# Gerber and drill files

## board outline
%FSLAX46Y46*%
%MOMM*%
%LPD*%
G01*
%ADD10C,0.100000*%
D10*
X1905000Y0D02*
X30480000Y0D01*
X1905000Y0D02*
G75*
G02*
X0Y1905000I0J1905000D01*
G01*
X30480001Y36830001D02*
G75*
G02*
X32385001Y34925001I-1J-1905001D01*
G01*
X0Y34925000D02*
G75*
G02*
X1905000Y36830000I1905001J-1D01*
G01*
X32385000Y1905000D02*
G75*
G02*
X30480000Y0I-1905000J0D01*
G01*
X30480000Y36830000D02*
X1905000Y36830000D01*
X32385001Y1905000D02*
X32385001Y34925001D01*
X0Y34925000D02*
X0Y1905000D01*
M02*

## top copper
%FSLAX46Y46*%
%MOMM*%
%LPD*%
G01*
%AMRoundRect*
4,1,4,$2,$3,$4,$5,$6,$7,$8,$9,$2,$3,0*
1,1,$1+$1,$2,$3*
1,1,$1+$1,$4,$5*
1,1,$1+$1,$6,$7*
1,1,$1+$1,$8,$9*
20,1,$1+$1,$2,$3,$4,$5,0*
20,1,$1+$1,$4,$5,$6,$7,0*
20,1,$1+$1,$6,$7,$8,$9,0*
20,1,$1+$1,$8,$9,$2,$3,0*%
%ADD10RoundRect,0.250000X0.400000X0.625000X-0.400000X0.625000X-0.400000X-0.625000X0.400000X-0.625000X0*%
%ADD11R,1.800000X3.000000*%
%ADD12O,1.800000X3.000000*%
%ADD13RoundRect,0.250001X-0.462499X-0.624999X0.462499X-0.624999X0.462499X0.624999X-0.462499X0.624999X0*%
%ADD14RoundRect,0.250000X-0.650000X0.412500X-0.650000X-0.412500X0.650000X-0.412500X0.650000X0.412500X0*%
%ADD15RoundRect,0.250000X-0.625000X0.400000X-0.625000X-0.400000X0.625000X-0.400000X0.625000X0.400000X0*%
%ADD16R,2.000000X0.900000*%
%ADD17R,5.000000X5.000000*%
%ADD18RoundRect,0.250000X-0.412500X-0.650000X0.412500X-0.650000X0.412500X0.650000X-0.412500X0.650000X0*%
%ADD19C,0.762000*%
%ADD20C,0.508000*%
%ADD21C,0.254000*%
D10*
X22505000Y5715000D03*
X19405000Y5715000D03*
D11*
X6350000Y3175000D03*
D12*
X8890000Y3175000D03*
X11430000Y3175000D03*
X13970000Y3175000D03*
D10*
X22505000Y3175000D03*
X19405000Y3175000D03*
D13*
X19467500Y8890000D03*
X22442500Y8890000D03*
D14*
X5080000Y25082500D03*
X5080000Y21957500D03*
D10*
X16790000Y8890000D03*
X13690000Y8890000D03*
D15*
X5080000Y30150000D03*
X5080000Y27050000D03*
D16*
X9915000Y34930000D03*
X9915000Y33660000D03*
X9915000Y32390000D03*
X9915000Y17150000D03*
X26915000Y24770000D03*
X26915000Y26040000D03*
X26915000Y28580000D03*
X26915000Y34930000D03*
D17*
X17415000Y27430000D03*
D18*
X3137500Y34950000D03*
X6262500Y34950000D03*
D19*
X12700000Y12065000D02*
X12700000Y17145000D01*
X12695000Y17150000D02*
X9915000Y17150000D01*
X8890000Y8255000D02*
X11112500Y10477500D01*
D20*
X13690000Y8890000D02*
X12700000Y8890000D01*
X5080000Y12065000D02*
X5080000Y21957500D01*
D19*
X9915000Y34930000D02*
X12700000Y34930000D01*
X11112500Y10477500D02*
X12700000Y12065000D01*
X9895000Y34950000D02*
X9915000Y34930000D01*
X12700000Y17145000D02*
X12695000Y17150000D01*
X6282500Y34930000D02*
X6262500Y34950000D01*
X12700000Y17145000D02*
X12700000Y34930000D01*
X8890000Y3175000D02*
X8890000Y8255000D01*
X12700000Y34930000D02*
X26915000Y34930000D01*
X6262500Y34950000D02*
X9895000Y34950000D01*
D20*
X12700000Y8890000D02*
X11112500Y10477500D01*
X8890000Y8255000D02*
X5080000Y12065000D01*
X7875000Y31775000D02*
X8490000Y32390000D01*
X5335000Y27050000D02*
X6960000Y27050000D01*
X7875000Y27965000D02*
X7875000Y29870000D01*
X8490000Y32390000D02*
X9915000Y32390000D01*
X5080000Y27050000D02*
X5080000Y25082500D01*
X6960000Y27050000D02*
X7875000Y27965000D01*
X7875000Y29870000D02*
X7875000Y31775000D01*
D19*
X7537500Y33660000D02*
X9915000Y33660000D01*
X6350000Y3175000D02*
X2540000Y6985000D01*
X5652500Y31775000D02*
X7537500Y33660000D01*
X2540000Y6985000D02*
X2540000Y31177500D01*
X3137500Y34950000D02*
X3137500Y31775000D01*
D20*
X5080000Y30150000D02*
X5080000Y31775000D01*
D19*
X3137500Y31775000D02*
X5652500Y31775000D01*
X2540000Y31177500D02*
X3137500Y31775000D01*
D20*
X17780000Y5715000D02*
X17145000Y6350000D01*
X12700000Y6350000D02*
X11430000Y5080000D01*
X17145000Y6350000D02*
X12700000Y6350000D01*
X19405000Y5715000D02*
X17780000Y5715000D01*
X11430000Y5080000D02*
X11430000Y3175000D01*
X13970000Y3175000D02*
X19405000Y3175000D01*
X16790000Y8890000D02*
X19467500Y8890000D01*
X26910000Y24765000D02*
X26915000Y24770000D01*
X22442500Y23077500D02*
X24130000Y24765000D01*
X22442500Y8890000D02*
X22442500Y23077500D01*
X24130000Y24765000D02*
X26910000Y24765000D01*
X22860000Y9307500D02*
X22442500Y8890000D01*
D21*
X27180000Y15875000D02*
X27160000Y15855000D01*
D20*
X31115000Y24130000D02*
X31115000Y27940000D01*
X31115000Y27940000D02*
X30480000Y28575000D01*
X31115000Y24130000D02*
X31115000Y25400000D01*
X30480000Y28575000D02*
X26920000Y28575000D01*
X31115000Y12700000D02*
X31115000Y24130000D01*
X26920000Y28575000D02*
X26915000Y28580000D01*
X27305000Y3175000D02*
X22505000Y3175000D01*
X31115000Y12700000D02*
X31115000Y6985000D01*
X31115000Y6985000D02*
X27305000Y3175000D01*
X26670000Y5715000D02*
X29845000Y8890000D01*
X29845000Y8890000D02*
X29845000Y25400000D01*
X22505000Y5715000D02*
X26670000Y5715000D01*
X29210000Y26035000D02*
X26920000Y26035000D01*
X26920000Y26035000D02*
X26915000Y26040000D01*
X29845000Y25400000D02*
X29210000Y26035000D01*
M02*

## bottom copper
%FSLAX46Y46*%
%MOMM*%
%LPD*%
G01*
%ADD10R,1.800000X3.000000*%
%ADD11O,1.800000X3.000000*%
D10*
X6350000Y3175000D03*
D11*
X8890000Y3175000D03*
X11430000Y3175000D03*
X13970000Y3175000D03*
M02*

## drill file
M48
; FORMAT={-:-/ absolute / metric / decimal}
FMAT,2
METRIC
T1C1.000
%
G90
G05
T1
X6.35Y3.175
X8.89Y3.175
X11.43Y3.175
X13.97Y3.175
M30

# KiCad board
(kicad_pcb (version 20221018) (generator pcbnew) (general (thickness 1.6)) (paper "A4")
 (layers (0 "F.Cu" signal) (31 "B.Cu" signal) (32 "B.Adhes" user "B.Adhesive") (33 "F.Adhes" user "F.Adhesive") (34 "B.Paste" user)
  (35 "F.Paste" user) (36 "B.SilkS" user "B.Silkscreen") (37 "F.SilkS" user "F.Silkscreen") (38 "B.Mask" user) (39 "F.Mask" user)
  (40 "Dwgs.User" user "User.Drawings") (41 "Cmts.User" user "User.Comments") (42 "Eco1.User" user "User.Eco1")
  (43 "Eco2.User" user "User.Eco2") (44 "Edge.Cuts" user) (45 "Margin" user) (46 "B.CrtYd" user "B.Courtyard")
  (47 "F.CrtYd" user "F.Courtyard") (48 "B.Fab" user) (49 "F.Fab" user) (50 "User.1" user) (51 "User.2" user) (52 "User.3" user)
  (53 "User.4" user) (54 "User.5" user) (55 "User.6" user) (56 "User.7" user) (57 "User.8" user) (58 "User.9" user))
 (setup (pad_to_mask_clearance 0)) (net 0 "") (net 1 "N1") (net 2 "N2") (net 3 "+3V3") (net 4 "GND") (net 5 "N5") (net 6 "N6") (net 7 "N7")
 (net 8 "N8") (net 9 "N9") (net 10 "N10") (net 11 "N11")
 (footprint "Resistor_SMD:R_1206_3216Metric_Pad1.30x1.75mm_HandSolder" (layer "F.Cu") (at 20.955 -5.715 180)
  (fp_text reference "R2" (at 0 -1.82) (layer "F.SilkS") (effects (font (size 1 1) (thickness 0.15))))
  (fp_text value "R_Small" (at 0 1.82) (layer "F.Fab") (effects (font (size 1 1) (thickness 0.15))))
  (pad "1" smd roundrect (at -1.55 0 180) (size 1.3 1.75) (layers "F.Cu" "F.Paste" "F.Mask") (roundrect_rratio 0.192308) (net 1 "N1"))
  (pad "2" smd roundrect (at 1.55 0 180) (size 1.3 1.75) (layers "F.Cu" "F.Paste" "F.Mask") (roundrect_rratio 0.192308) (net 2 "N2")))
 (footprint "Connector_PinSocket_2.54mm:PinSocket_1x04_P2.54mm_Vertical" (layer "F.Cu") (at 6.35 -3.175 90)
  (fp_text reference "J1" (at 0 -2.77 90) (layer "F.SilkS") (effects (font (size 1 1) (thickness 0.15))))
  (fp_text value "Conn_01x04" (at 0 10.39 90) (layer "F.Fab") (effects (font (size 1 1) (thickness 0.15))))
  (pad "1" thru_hole rect (at 0 0 90) (size 3 1.8) (drill 1) (layers "*.Cu" "*.Mask") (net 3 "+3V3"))
  (pad "2" thru_hole oval (at 0 2.54 90) (size 3 1.8) (drill 1) (layers "*.Cu" "*.Mask") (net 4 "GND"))
  (pad "3" thru_hole oval (at 0 5.08 90) (size 3 1.8) (drill 1) (layers "*.Cu" "*.Mask") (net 2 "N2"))
  (pad "4" thru_hole oval (at 0 7.62 90) (size 3 1.8) (drill 1) (layers "*.Cu" "*.Mask") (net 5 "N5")))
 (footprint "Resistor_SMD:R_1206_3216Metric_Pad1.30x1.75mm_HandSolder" (layer "F.Cu") (at 20.955 -3.175 180)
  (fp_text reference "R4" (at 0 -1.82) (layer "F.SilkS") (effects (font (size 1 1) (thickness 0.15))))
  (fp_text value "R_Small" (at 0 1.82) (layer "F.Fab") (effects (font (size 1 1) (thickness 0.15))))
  (pad "1" smd roundrect (at -1.55 0 180) (size 1.3 1.75) (layers "F.Cu" "F.Paste" "F.Mask") (roundrect_rratio 0.192308) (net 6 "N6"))
  (pad "2" smd roundrect (at 1.55 0 180) (size 1.3 1.75) (layers "F.Cu" "F.Paste" "F.Mask") (roundrect_rratio 0.192308) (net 5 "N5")))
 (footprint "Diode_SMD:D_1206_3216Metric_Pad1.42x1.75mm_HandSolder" (layer "F.Cu") (at 20.955 -8.89)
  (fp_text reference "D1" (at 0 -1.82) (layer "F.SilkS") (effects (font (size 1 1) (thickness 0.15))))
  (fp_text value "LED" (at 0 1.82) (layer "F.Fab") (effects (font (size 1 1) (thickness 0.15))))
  (pad "1" smd roundrect (at -1.4875 0) (size 1.425 1.75) (layers "F.Cu" "F.Paste" "F.Mask") (roundrect_rratio 0.175439) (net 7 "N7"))
  (pad "2" smd roundrect (at 1.4875 0) (size 1.425 1.75) (layers "F.Cu" "F.Paste" "F.Mask") (roundrect_rratio 0.175439) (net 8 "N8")))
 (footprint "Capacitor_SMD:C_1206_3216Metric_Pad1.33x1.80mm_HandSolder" (layer "F.Cu") (at 5.08 -23.52 -90)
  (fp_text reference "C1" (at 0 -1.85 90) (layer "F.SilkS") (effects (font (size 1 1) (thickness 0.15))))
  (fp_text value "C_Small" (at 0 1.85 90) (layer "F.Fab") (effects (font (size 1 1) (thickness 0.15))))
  (pad "1" smd roundrect (at -1.5625 0 270) (size 1.325 1.8) (layers "F.Cu" "F.Paste" "F.Mask") (roundrect_rratio 0.1886792453) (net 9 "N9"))
  (pad "2" smd roundrect (at 1.5625 0 270) (size 1.325 1.8) (layers "F.Cu" "F.Paste" "F.Mask") (roundrect_rratio 0.1886792453) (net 4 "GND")))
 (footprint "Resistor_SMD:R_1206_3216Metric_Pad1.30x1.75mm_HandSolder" (layer "F.Cu") (at 15.24 -8.89 180)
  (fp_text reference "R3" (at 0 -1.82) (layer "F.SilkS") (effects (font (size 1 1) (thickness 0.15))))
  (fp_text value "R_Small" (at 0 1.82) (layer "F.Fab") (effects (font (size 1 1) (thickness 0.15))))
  (pad "1" smd roundrect (at -1.55 0 180) (size 1.3 1.75) (layers "F.Cu" "F.Paste" "F.Mask") (roundrect_rratio 0.192308) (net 7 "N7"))
  (pad "2" smd roundrect (at 1.55 0 180) (size 1.3 1.75) (layers "F.Cu" "F.Paste" "F.Mask") (roundrect_rratio 0.192308) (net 4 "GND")))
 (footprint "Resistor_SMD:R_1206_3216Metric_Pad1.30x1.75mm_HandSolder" (layer "F.Cu") (at 5.08 -28.6 -90)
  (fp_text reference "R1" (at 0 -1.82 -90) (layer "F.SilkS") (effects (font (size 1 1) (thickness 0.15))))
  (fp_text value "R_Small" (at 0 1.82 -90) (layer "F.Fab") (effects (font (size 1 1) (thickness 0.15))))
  (pad "1" smd roundrect (at -1.55 0 270) (size 1.3 1.75) (layers "F.Cu" "F.Paste" "F.Mask") (roundrect_rratio 0.192308) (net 3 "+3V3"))
  (pad "2" smd roundrect (at 1.55 0 270) (size 1.3 1.75) (layers "F.Cu" "F.Paste" "F.Mask") (roundrect_rratio 0.192308) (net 9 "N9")))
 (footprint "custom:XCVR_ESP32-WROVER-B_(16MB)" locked (layer "F.Cu") (at 18.415 -26.67)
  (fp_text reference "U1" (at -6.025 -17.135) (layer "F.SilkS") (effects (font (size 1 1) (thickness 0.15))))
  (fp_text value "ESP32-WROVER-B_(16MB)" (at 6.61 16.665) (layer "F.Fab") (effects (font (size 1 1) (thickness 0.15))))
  (pad "1" smd rect locked (at -8.5 -8.26) (size 2 0.9) (layers "F.Cu" "F.Paste" "F.Mask") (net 4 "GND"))
  (pad "2" smd rect locked (at -8.5 -6.99) (size 2 0.9) (layers "F.Cu" "F.Paste" "F.Mask") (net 3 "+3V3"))
  (pad "3" smd rect locked (at -8.5 -5.72) (size 2 0.9) (layers "F.Cu" "F.Paste" "F.Mask") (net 9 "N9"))
  (pad "15" smd rect locked (at -8.5 9.52) (size 2 0.9) (layers "F.Cu" "F.Paste" "F.Mask") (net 4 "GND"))
  (pad "30" smd rect locked (at 8.5 1.9) (size 2 0.9) (layers "F.Cu" "F.Paste" "F.Mask") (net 8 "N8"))
  (pad "31" smd rect locked (at 8.5 0.63) (size 2 0.9) (layers "F.Cu" "F.Paste" "F.Mask") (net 1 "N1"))
  (pad "33" smd rect locked (at 8.5 -1.91) (size 2 0.9) (layers "F.Cu" "F.Paste" "F.Mask") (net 6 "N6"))
  (pad "38" smd rect locked (at 8.5 -8.26) (size 2 0.9) (layers "F.Cu" "F.Paste" "F.Mask") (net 4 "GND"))
  (pad "39" smd rect locked (at -1 -0.76) (size 5 5) (layers "F.Cu" "F.Mask") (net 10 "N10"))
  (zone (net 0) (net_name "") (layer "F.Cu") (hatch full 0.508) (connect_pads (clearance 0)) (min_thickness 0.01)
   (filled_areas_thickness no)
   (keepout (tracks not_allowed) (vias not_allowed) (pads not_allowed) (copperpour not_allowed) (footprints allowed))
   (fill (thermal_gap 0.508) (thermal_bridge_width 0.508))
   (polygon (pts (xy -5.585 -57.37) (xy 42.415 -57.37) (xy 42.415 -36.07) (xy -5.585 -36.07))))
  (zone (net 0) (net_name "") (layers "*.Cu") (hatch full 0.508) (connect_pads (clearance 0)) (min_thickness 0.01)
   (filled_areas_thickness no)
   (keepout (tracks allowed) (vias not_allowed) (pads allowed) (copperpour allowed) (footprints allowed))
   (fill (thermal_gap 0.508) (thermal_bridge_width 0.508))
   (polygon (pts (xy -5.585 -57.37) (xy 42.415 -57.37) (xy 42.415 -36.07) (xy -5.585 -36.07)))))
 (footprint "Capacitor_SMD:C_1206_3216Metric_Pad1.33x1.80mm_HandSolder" (layer "F.Cu") (at 4.7 -34.95)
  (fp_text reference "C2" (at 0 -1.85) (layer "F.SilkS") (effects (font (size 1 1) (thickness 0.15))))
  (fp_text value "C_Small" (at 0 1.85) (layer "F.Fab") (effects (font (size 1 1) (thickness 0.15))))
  (pad "1" smd roundrect (at -1.5625 0) (size 1.325 1.8) (layers "F.Cu" "F.Paste" "F.Mask") (roundrect_rratio 0.1886792453) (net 3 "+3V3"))
  (pad "2" smd roundrect (at 1.5625 0) (size 1.325 1.8) (layers "F.Cu" "F.Paste" "F.Mask") (roundrect_rratio 0.1886792453) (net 4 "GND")))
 (gr_line (start 1.905 0) (end 30.48 0) (stroke (width 0.1) (type default)) (layer "Edge.Cuts"))
 (gr_arc (start 1.905 0) (mid 0.557962 -0.557962) (end 0 -1.905) (stroke (width 0.1) (type default)) (layer "Edge.Cuts"))
 (gr_arc (start 30.480001 -36.830001) (mid 31.827039 -36.272039) (end 32.385001 -34.925001) (stroke (width 0.1) (type default))
  (layer "Edge.Cuts"))
 (gr_arc (start 0 -34.925) (mid 0.557962 -36.272038) (end 1.905 -36.83) (stroke (width 0.1) (type default)) (layer "Edge.Cuts"))
 (gr_arc (start 32.385 -1.905) (mid 31.827038 -0.557962) (end 30.48 0) (stroke (width 0.1) (type default)) (layer "Edge.Cuts"))
 (gr_line (start 30.48 -36.83) (end 1.905 -36.83) (stroke (width 0.1) (type default)) (layer "Edge.Cuts"))
 (gr_line (start 32.385001 -1.905) (end 32.385001 -34.925001) (stroke (width 0.1) (type default)) (layer "Edge.Cuts"))
 (gr_line (start 0 -34.925) (end 0 -1.905) (stroke (width 0.1) (type default)) (layer "Edge.Cuts"))
 (segment (start 12.7 -12.065) (end 12.7 -17.145) (width 0.762) (layer "F.Cu") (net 4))
 (segment (start 12.695 -17.15) (end 9.915 -17.15) (width 0.762) (layer "F.Cu") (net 4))
 (segment (start 8.89 -8.255) (end 11.1125 -10.4775) (width 0.762) (layer "F.Cu") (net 4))
 (segment (start 13.69 -8.89) (end 12.7 -8.89) (width 0.508) (layer "F.Cu") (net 4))
 (segment (start 5.08 -12.065) (end 5.08 -21.9575) (width 0.508) (layer "F.Cu") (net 4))
 (segment (start 9.915 -34.93) (end 12.7 -34.93) (width 0.762) (layer "F.Cu") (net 4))
 (segment (start 11.1125 -10.4775) (end 12.7 -12.065) (width 0.762) (layer "F.Cu") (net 4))
 (segment (start 9.895 -34.95) (end 9.915 -34.93) (width 0.762) (layer "F.Cu") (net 4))
 (segment (start 12.7 -17.145) (end 12.695 -17.15) (width 0.762) (layer "F.Cu") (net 4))
 (segment (start 6.2825 -34.93) (end 6.2625 -34.95) (width 0.762) (layer "F.Cu") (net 4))
 (segment (start 12.7 -17.145) (end 12.7 -34.93) (width 0.762) (layer "F.Cu") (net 4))
 (segment (start 8.89 -3.175) (end 8.89 -8.255) (width 0.762) (layer "F.Cu") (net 4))
 (segment (start 12.7 -34.93) (end 26.915 -34.93) (width 0.762) (layer "F.Cu") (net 4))
 (segment (start 6.2625 -34.95) (end 9.895 -34.95) (width 0.762) (layer "F.Cu") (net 4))
 (segment (start 12.7 -8.89) (end 11.1125 -10.4775) (width 0.508) (layer "F.Cu") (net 4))
 (segment (start 8.89 -8.255) (end 5.08 -12.065) (width 0.508) (layer "F.Cu") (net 4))
 (segment (start 7.875 -31.775) (end 8.49 -32.39) (width 0.508) (layer "F.Cu") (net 9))
 (segment (start 5.335 -27.05) (end 6.96 -27.05) (width 0.508) (layer "F.Cu") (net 9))
 (segment (start 7.875 -27.965) (end 7.875 -29.87) (width 0.508) (layer "F.Cu") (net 9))
 (segment (start 8.49 -32.39) (end 9.915 -32.39) (width 0.508) (layer "F.Cu") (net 9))
 (segment (start 5.08 -27.05) (end 5.08 -25.0825) (width 0.508) (layer "F.Cu") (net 9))
 (segment (start 6.96 -27.05) (end 7.875 -27.965) (width 0.508) (layer "F.Cu") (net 9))
 (segment (start 7.875 -29.87) (end 7.875 -31.775) (width 0.508) (layer "F.Cu") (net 9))
 (segment (start 7.5375 -33.66) (end 9.915 -33.66) (width 0.762) (layer "F.Cu") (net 3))
 (segment (start 6.35 -3.175) (end 2.54 -6.985) (width 0.762) (layer "F.Cu") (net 3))
 (segment (start 5.6525 -31.775) (end 7.5375 -33.66) (width 0.762) (layer "F.Cu") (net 3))
 (segment (start 2.54 -6.985) (end 2.54 -31.1775) (width 0.762) (layer "F.Cu") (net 3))
 (segment (start 3.1375 -34.95) (end 3.1375 -31.775) (width 0.762) (layer "F.Cu") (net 3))
 (segment (start 5.08 -30.15) (end 5.08 -31.775) (width 0.508) (layer "F.Cu") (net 3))
 (segment (start 3.1375 -31.775) (end 5.6525 -31.775) (width 0.762) (layer "F.Cu") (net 3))
 (segment (start 2.54 -31.1775) (end 3.1375 -31.775) (width 0.762) (layer "F.Cu") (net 3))
 (segment (start 17.78 -5.715) (end 17.145 -6.35) (width 0.508) (layer "F.Cu") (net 2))
 (segment (start 12.7 -6.35) (end 11.43 -5.08) (width 0.508) (layer "F.Cu") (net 2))
 (segment (start 17.145 -6.35) (end 12.7 -6.35) (width 0.508) (layer "F.Cu") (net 2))
 (segment (start 19.405 -5.715) (end 17.78 -5.715) (width 0.508) (layer "F.Cu") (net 2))
 (segment (start 11.43 -5.08) (end 11.43 -3.175) (width 0.508) (layer "F.Cu") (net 2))
 (segment (start 13.97 -3.175) (end 19.405 -3.175) (width 0.508) (layer "F.Cu") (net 5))
 (segment (start 16.79 -8.89) (end 19.4675 -8.89) (width 0.508) (layer "F.Cu") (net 7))
 (segment (start 26.91 -24.765) (end 26.915 -24.77) (width 0.508) (layer "F.Cu") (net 8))
 (segment (start 22.4425 -23.0775) (end 24.13 -24.765) (width 0.508) (layer "F.Cu") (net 8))
 (segment (start 22.4425 -8.89) (end 22.4425 -23.0775) (width 0.508) (layer "F.Cu") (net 8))
 (segment (start 24.13 -24.765) (end 26.91 -24.765) (width 0.508) (layer "F.Cu") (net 8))
 (segment (start 22.86 -9.3075) (end 22.4425 -8.89) (width 0.508) (layer "F.Cu") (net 8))
 (segment (start 27.18 -15.875) (end 27.16 -15.855) (width 0.254) (layer "F.Cu") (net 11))
 (segment (start 31.115 -24.13) (end 31.115 -27.94) (width 0.508) (layer "F.Cu") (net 6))
 (segment (start 31.115 -27.94) (end 30.48 -28.575) (width 0.508) (layer "F.Cu") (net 6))
 (segment (start 31.115 -24.13) (end 31.115 -25.4) (width 0.508) (layer "F.Cu") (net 6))
 (segment (start 30.48 -28.575) (end 26.92 -28.575) (width 0.508) (layer "F.Cu") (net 6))
 (segment (start 31.115 -12.7) (end 31.115 -24.13) (width 0.508) (layer "F.Cu") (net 6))
 (segment (start 26.92 -28.575) (end 26.915 -28.58) (width 0.508) (layer "F.Cu") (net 6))
 (segment (start 27.305 -3.175) (end 22.505 -3.175) (width 0.508) (layer "F.Cu") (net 6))
 (segment (start 31.115 -12.7) (end 31.115 -6.985) (width 0.508) (layer "F.Cu") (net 6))
 (segment (start 31.115 -6.985) (end 27.305 -3.175) (width 0.508) (layer "F.Cu") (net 6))
 (segment (start 26.67 -5.715) (end 29.845 -8.89) (width 0.508) (layer "F.Cu") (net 1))
 (segment (start 29.845 -8.89) (end 29.845 -25.4) (width 0.508) (layer "F.Cu") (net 1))
 (segment (start 22.505 -5.715) (end 26.67 -5.715) (width 0.508) (layer "F.Cu") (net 1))
 (segment (start 29.21 -26.035) (end 26.92 -26.035) (width 0.508) (layer "F.Cu") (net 1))
 (segment (start 26.92 -26.035) (end 26.915 -26.04) (width 0.508) (layer "F.Cu") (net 1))
 (segment (start 29.845 -25.4) (end 29.21 -26.035) (width 0.508) (layer "F.Cu") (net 1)))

